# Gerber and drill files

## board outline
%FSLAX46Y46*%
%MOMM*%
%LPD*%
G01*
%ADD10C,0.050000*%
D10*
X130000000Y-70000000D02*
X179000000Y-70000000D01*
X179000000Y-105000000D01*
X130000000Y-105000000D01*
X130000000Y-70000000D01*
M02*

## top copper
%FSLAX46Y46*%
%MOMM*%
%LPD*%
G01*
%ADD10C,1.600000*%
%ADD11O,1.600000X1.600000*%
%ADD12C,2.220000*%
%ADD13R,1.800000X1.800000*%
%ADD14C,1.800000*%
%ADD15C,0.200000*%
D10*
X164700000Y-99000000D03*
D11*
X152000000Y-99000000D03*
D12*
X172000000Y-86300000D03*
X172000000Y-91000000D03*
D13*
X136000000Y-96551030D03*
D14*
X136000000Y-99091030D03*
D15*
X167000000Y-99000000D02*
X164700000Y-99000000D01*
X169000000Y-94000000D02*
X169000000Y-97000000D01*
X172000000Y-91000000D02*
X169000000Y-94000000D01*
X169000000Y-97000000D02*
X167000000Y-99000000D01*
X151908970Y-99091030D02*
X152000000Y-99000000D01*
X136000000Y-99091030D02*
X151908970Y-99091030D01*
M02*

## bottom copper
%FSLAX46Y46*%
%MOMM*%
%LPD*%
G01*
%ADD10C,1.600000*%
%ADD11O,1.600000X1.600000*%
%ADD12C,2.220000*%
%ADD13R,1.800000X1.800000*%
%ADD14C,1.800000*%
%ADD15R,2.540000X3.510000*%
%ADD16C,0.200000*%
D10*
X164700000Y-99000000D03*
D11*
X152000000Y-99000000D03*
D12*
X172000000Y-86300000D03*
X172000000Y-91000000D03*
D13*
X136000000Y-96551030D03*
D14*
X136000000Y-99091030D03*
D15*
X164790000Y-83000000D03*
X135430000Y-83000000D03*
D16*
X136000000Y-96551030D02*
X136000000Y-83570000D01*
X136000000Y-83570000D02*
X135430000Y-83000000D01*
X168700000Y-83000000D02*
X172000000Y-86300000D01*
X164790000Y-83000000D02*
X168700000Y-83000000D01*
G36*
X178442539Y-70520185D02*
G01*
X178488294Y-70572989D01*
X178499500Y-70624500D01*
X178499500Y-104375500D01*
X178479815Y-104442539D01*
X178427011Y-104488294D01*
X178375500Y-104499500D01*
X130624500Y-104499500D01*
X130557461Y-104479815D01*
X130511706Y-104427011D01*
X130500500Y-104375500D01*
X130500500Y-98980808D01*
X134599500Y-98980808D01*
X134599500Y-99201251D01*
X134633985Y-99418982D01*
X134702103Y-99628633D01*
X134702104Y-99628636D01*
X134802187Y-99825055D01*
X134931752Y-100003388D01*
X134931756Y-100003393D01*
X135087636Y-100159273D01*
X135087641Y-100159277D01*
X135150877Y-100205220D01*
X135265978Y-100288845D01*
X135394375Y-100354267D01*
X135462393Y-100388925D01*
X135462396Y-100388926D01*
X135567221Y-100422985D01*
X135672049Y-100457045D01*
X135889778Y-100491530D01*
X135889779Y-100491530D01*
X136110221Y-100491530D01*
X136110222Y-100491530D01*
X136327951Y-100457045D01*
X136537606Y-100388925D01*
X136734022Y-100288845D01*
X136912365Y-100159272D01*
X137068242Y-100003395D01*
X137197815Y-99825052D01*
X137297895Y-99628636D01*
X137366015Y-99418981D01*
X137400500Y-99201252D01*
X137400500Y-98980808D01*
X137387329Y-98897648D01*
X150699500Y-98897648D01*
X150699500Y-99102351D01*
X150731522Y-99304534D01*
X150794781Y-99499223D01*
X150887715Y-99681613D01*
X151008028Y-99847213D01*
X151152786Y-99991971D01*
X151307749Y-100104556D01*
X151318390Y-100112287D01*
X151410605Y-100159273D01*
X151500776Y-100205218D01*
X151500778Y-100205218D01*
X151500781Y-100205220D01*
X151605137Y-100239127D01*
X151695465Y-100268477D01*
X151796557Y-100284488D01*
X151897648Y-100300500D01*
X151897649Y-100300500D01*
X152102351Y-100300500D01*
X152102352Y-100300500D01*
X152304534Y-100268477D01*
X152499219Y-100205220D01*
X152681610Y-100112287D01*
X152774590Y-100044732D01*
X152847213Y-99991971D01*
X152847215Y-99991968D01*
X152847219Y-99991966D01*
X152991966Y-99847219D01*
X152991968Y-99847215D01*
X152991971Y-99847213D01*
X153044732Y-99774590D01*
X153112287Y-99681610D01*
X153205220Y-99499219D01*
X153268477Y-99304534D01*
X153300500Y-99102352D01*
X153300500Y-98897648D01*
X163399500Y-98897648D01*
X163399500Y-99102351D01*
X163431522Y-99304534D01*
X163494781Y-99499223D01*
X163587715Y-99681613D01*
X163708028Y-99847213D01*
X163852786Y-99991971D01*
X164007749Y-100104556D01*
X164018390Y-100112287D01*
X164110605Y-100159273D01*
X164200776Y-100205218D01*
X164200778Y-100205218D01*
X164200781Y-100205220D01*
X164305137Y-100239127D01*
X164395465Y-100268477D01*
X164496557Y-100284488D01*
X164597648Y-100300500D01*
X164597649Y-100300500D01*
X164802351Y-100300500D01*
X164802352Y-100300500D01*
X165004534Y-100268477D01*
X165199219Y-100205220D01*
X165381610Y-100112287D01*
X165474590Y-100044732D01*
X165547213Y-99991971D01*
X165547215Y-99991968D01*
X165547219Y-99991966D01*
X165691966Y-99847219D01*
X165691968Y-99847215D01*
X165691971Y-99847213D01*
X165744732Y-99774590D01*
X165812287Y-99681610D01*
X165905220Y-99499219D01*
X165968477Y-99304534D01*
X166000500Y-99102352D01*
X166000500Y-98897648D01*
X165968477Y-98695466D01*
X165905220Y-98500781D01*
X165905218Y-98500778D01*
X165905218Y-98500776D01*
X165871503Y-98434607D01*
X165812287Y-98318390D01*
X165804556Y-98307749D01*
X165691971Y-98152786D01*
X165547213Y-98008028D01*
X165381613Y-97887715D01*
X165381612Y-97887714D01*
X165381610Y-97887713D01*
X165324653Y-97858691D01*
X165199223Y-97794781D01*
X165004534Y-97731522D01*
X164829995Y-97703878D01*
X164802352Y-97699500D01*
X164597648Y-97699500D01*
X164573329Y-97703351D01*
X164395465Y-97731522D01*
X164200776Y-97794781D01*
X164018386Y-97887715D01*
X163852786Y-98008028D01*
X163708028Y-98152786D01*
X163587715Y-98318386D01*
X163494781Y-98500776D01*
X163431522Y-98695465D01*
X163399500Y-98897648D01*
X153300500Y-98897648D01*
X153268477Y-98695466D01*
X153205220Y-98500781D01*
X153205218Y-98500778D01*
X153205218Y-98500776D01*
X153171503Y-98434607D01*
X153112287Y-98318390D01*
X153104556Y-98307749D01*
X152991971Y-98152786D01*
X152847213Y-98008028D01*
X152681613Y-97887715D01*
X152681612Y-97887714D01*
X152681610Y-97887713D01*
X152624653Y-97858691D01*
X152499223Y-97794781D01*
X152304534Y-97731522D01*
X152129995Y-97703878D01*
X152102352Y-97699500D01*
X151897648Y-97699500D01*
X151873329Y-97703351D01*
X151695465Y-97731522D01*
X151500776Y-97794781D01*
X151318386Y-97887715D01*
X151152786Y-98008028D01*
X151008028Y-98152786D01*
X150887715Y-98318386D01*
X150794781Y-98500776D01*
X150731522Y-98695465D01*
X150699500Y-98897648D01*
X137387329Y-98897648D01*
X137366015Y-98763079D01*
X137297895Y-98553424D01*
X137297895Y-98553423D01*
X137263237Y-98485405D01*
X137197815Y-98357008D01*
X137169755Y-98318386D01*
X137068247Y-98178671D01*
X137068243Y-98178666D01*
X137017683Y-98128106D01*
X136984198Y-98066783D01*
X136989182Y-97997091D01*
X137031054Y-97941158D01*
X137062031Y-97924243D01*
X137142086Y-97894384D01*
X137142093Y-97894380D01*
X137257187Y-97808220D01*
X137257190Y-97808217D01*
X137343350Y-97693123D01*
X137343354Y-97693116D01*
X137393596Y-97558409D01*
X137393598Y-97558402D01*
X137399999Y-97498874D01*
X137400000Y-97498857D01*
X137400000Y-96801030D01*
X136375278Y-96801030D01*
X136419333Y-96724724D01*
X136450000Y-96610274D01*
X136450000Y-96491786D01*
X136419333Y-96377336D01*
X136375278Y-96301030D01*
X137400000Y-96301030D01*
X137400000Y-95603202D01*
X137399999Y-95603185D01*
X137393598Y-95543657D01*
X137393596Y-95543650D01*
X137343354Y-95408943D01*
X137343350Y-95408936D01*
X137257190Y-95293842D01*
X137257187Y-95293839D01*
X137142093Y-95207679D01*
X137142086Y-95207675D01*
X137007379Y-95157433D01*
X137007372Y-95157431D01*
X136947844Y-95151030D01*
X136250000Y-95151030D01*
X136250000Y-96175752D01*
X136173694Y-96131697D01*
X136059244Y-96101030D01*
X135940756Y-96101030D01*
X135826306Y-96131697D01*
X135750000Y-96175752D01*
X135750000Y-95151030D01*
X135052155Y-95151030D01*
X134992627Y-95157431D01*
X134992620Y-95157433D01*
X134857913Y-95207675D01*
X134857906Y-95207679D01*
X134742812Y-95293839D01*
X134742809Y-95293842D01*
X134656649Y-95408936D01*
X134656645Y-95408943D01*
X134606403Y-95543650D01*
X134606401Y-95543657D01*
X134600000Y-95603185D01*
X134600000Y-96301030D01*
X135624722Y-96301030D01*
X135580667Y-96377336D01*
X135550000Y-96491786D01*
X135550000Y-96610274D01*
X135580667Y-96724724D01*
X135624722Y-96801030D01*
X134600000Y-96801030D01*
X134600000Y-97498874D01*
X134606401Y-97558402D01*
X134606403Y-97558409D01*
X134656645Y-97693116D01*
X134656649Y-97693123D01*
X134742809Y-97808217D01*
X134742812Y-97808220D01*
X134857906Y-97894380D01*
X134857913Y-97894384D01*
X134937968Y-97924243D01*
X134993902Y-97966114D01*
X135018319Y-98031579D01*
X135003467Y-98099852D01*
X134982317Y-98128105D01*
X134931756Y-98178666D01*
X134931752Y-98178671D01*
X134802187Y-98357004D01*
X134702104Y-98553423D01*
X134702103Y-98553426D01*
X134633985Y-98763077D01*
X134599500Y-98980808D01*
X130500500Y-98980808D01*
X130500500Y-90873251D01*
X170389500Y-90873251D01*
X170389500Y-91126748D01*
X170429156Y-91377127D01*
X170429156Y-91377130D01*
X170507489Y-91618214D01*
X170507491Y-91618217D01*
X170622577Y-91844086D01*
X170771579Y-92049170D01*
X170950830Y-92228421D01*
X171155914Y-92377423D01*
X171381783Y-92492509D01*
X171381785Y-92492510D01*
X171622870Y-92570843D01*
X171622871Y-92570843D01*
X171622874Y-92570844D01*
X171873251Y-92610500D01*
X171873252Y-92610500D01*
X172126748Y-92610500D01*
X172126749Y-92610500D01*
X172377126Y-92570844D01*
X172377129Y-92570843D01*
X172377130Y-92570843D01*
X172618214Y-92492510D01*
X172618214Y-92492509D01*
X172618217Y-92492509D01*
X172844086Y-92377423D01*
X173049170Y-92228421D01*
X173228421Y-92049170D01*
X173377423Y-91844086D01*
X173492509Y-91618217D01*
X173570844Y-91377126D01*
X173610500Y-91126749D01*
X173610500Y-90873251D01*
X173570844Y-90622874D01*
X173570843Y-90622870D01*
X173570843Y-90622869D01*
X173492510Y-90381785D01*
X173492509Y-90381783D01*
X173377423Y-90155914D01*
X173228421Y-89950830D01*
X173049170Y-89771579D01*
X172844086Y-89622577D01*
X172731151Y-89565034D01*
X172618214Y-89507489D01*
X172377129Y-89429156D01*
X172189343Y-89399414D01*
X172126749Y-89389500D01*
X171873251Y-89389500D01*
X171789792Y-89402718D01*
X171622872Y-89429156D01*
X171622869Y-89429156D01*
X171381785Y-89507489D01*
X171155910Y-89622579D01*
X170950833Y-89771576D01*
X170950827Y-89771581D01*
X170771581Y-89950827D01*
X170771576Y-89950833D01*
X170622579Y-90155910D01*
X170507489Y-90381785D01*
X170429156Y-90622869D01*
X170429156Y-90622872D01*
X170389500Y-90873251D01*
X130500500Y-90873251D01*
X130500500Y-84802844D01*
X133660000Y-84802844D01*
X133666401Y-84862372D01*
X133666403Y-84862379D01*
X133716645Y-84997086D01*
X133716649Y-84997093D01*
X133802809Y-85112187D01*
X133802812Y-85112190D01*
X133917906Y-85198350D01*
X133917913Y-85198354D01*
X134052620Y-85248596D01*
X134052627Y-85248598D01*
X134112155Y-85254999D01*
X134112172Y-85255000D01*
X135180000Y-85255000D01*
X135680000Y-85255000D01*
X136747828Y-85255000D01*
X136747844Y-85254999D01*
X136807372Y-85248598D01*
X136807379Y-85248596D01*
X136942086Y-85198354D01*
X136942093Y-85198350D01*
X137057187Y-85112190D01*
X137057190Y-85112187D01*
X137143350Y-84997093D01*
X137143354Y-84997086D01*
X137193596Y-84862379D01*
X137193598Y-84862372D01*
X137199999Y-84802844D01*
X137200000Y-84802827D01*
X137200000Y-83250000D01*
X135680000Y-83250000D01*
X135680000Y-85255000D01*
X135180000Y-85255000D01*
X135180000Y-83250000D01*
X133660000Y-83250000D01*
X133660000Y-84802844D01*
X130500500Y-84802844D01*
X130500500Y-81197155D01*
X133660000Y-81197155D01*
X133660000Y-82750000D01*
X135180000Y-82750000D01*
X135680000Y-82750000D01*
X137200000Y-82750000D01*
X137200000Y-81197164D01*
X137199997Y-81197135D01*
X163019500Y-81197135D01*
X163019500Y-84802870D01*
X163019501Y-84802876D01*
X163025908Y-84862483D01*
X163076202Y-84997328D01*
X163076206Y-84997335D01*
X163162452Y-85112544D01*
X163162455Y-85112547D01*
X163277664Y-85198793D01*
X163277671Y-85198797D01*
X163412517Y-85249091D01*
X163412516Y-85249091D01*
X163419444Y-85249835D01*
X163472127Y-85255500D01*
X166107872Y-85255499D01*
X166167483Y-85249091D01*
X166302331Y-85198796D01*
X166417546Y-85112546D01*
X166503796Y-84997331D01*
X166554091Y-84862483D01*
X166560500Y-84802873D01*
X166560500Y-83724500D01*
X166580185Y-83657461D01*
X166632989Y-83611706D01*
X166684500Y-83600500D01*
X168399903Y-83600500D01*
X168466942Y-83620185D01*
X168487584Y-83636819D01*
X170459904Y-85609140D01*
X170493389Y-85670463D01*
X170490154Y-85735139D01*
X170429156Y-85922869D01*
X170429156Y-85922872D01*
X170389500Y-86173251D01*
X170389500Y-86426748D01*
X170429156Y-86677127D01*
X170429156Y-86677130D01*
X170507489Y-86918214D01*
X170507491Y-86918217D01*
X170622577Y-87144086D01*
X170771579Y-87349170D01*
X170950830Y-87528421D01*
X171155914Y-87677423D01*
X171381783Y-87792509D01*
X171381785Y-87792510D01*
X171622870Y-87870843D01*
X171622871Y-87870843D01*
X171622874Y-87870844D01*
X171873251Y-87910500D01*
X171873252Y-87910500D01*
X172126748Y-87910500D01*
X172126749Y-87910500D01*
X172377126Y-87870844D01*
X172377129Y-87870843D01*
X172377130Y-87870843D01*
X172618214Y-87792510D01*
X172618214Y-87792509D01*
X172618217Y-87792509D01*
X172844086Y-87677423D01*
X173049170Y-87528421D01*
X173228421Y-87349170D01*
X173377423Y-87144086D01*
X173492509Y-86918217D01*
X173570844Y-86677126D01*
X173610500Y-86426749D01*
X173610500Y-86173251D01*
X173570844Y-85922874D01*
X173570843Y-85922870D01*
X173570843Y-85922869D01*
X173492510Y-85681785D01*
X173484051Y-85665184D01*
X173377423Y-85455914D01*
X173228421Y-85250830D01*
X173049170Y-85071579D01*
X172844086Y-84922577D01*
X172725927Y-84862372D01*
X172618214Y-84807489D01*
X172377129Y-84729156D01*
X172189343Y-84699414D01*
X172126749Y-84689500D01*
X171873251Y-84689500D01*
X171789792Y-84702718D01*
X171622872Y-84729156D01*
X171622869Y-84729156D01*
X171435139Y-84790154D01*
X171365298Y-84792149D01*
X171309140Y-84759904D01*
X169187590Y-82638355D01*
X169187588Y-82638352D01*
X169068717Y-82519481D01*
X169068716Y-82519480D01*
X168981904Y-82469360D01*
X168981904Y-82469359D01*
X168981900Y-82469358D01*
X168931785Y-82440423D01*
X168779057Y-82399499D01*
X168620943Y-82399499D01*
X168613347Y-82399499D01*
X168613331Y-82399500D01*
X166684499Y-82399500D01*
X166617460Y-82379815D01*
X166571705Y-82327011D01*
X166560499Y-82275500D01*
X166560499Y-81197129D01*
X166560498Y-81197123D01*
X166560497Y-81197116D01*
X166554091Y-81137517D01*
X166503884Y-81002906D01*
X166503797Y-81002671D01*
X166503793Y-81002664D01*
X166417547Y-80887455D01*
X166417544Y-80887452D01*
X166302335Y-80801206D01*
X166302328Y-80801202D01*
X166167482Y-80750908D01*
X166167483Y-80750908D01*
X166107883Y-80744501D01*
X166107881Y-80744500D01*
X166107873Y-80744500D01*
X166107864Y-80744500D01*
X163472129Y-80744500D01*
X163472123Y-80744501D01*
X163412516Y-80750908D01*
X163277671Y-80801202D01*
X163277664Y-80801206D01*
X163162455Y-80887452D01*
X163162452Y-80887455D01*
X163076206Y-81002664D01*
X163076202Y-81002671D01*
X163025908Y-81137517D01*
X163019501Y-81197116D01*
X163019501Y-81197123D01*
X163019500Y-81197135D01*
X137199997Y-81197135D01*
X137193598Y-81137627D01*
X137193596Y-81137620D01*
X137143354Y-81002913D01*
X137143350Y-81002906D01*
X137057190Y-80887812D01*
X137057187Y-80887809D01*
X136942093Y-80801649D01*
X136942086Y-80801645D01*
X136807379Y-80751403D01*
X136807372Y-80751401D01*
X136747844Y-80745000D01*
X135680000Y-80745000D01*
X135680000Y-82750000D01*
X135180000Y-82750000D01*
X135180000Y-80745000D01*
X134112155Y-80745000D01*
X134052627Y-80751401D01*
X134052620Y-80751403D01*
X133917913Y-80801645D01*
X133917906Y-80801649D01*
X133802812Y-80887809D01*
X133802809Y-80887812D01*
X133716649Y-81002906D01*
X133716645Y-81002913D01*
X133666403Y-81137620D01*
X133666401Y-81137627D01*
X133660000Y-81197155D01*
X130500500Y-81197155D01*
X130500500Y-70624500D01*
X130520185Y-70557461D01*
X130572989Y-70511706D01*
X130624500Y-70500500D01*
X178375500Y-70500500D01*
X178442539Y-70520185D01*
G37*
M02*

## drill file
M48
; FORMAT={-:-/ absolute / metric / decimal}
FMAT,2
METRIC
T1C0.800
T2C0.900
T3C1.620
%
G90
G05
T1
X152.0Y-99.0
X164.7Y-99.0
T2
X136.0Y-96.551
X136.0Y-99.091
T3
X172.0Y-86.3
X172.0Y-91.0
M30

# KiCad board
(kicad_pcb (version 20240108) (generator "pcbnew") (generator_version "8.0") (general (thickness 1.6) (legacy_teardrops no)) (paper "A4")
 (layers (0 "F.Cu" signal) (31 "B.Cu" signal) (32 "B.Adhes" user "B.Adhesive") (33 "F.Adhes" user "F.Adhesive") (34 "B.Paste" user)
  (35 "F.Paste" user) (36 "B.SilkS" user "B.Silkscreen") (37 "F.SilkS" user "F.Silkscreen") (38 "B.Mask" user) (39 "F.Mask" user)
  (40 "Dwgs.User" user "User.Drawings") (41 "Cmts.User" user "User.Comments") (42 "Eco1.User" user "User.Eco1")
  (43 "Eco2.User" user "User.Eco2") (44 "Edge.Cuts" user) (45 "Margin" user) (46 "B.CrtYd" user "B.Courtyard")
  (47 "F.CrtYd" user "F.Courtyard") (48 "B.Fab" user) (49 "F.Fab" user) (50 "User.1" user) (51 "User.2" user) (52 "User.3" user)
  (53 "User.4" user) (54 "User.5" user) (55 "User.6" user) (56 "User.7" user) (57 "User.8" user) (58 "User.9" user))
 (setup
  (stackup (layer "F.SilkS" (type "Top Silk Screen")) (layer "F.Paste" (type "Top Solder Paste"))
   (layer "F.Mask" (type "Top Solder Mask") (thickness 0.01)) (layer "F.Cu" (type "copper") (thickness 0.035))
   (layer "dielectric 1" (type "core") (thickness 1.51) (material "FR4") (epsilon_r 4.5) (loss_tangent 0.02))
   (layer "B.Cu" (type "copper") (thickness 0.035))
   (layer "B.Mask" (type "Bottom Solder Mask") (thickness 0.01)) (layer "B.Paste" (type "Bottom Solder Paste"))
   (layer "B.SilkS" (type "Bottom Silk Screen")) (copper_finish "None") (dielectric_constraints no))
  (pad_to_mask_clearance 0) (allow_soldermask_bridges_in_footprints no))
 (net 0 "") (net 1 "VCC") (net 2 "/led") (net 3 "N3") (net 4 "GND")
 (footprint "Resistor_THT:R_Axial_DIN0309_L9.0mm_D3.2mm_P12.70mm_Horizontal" (layer "F.Cu") (at 164.7 99 180)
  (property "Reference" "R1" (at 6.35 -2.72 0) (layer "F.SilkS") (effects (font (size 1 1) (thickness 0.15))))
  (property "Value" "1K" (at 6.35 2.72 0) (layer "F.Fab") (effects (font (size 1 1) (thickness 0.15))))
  (pad "1" thru_hole circle (at 0 0 180) (size 1.6 1.6) (drill 0.8) (layers "*.Cu" "*.Mask") (remove_unused_layers no) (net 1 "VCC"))
  (pad "2" thru_hole oval (at 12.7 0 180) (size 1.6 1.6) (drill 0.8) (layers "*.Cu" "*.Mask") (remove_unused_layers no) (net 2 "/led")))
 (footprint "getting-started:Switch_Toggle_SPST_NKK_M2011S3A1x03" (layer "F.Cu") (at 172 81.6)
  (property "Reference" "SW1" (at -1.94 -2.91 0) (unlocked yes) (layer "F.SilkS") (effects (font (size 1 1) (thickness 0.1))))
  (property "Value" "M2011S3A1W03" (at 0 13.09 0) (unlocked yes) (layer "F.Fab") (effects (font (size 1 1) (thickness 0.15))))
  (pad "2" thru_hole circle (at 0 4.7) (size 2.22 2.22) (drill 1.62) (layers "*.Cu" "*.Mask") (remove_unused_layers no) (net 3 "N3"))
  (pad "3" thru_hole circle (at 0 9.4) (size 2.22 2.22) (drill 1.62) (layers "*.Cu" "*.Mask") (remove_unused_layers no) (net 1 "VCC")))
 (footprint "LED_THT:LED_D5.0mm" (layer "F.Cu") (at 136 96.55103 -90)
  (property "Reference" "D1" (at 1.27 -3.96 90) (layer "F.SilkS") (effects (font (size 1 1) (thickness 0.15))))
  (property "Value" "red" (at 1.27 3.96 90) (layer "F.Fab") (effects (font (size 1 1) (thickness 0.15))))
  (pad "1" thru_hole rect (at 0 0 270) (size 1.8 1.8) (drill 0.9) (layers "*.Cu" "*.Mask") (remove_unused_layers no) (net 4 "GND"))
  (pad "2" thru_hole circle (at 2.54 0 270) (size 1.8 1.8) (drill 0.9) (layers "*.Cu" "*.Mask") (remove_unused_layers no) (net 2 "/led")))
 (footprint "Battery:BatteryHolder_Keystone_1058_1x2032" (layer "B.Cu") (at 150.11 83 180)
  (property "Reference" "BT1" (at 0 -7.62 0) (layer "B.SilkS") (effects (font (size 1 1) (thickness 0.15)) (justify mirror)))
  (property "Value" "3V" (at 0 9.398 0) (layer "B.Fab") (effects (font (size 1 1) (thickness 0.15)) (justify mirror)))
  (pad "1" smd rect (at -14.68 0 180) (size 2.54 3.51) (layers "B.Cu" "B.Paste" "B.Mask") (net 3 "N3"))
  (pad "2" smd rect (at 14.68 0 180) (size 2.54 3.51) (layers "B.Cu" "B.Paste" "B.Mask") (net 4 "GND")))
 (gr_rect (start 130 70) (end 179 105) (stroke (width 0.05) (type default)) (fill none) (layer "Edge.Cuts"))
 (segment (start 136 96.55103) (end 136 83.57) (width 0.2) (layer "B.Cu") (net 4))
 (segment (start 136 83.57) (end 135.43 83) (width 0.2) (layer "B.Cu") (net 4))
 (segment (start 167 99) (end 164.7 99) (width 0.2) (layer "F.Cu") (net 1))
 (segment (start 169 94) (end 169 97) (width 0.2) (layer "F.Cu") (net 1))
 (segment (start 172 91) (end 169 94) (width 0.2) (layer "F.Cu") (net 1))
 (segment (start 169 97) (end 167 99) (width 0.2) (layer "F.Cu") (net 1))
 (segment (start 151.90897 99.09103) (end 152 99) (width 0.2) (layer "F.Cu") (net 2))
 (segment (start 136 99.09103) (end 151.90897 99.09103) (width 0.2) (layer "F.Cu") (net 2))
 (segment (start 168.7 83) (end 172 86.3) (width 0.2) (layer "B.Cu") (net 3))
 (segment (start 164.79 83) (end 168.7 83) (width 0.2) (layer "B.Cu") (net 3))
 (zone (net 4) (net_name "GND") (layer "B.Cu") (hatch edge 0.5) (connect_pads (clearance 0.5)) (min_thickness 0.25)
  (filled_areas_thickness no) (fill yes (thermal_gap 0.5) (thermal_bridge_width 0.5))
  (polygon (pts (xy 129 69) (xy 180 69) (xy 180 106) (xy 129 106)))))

